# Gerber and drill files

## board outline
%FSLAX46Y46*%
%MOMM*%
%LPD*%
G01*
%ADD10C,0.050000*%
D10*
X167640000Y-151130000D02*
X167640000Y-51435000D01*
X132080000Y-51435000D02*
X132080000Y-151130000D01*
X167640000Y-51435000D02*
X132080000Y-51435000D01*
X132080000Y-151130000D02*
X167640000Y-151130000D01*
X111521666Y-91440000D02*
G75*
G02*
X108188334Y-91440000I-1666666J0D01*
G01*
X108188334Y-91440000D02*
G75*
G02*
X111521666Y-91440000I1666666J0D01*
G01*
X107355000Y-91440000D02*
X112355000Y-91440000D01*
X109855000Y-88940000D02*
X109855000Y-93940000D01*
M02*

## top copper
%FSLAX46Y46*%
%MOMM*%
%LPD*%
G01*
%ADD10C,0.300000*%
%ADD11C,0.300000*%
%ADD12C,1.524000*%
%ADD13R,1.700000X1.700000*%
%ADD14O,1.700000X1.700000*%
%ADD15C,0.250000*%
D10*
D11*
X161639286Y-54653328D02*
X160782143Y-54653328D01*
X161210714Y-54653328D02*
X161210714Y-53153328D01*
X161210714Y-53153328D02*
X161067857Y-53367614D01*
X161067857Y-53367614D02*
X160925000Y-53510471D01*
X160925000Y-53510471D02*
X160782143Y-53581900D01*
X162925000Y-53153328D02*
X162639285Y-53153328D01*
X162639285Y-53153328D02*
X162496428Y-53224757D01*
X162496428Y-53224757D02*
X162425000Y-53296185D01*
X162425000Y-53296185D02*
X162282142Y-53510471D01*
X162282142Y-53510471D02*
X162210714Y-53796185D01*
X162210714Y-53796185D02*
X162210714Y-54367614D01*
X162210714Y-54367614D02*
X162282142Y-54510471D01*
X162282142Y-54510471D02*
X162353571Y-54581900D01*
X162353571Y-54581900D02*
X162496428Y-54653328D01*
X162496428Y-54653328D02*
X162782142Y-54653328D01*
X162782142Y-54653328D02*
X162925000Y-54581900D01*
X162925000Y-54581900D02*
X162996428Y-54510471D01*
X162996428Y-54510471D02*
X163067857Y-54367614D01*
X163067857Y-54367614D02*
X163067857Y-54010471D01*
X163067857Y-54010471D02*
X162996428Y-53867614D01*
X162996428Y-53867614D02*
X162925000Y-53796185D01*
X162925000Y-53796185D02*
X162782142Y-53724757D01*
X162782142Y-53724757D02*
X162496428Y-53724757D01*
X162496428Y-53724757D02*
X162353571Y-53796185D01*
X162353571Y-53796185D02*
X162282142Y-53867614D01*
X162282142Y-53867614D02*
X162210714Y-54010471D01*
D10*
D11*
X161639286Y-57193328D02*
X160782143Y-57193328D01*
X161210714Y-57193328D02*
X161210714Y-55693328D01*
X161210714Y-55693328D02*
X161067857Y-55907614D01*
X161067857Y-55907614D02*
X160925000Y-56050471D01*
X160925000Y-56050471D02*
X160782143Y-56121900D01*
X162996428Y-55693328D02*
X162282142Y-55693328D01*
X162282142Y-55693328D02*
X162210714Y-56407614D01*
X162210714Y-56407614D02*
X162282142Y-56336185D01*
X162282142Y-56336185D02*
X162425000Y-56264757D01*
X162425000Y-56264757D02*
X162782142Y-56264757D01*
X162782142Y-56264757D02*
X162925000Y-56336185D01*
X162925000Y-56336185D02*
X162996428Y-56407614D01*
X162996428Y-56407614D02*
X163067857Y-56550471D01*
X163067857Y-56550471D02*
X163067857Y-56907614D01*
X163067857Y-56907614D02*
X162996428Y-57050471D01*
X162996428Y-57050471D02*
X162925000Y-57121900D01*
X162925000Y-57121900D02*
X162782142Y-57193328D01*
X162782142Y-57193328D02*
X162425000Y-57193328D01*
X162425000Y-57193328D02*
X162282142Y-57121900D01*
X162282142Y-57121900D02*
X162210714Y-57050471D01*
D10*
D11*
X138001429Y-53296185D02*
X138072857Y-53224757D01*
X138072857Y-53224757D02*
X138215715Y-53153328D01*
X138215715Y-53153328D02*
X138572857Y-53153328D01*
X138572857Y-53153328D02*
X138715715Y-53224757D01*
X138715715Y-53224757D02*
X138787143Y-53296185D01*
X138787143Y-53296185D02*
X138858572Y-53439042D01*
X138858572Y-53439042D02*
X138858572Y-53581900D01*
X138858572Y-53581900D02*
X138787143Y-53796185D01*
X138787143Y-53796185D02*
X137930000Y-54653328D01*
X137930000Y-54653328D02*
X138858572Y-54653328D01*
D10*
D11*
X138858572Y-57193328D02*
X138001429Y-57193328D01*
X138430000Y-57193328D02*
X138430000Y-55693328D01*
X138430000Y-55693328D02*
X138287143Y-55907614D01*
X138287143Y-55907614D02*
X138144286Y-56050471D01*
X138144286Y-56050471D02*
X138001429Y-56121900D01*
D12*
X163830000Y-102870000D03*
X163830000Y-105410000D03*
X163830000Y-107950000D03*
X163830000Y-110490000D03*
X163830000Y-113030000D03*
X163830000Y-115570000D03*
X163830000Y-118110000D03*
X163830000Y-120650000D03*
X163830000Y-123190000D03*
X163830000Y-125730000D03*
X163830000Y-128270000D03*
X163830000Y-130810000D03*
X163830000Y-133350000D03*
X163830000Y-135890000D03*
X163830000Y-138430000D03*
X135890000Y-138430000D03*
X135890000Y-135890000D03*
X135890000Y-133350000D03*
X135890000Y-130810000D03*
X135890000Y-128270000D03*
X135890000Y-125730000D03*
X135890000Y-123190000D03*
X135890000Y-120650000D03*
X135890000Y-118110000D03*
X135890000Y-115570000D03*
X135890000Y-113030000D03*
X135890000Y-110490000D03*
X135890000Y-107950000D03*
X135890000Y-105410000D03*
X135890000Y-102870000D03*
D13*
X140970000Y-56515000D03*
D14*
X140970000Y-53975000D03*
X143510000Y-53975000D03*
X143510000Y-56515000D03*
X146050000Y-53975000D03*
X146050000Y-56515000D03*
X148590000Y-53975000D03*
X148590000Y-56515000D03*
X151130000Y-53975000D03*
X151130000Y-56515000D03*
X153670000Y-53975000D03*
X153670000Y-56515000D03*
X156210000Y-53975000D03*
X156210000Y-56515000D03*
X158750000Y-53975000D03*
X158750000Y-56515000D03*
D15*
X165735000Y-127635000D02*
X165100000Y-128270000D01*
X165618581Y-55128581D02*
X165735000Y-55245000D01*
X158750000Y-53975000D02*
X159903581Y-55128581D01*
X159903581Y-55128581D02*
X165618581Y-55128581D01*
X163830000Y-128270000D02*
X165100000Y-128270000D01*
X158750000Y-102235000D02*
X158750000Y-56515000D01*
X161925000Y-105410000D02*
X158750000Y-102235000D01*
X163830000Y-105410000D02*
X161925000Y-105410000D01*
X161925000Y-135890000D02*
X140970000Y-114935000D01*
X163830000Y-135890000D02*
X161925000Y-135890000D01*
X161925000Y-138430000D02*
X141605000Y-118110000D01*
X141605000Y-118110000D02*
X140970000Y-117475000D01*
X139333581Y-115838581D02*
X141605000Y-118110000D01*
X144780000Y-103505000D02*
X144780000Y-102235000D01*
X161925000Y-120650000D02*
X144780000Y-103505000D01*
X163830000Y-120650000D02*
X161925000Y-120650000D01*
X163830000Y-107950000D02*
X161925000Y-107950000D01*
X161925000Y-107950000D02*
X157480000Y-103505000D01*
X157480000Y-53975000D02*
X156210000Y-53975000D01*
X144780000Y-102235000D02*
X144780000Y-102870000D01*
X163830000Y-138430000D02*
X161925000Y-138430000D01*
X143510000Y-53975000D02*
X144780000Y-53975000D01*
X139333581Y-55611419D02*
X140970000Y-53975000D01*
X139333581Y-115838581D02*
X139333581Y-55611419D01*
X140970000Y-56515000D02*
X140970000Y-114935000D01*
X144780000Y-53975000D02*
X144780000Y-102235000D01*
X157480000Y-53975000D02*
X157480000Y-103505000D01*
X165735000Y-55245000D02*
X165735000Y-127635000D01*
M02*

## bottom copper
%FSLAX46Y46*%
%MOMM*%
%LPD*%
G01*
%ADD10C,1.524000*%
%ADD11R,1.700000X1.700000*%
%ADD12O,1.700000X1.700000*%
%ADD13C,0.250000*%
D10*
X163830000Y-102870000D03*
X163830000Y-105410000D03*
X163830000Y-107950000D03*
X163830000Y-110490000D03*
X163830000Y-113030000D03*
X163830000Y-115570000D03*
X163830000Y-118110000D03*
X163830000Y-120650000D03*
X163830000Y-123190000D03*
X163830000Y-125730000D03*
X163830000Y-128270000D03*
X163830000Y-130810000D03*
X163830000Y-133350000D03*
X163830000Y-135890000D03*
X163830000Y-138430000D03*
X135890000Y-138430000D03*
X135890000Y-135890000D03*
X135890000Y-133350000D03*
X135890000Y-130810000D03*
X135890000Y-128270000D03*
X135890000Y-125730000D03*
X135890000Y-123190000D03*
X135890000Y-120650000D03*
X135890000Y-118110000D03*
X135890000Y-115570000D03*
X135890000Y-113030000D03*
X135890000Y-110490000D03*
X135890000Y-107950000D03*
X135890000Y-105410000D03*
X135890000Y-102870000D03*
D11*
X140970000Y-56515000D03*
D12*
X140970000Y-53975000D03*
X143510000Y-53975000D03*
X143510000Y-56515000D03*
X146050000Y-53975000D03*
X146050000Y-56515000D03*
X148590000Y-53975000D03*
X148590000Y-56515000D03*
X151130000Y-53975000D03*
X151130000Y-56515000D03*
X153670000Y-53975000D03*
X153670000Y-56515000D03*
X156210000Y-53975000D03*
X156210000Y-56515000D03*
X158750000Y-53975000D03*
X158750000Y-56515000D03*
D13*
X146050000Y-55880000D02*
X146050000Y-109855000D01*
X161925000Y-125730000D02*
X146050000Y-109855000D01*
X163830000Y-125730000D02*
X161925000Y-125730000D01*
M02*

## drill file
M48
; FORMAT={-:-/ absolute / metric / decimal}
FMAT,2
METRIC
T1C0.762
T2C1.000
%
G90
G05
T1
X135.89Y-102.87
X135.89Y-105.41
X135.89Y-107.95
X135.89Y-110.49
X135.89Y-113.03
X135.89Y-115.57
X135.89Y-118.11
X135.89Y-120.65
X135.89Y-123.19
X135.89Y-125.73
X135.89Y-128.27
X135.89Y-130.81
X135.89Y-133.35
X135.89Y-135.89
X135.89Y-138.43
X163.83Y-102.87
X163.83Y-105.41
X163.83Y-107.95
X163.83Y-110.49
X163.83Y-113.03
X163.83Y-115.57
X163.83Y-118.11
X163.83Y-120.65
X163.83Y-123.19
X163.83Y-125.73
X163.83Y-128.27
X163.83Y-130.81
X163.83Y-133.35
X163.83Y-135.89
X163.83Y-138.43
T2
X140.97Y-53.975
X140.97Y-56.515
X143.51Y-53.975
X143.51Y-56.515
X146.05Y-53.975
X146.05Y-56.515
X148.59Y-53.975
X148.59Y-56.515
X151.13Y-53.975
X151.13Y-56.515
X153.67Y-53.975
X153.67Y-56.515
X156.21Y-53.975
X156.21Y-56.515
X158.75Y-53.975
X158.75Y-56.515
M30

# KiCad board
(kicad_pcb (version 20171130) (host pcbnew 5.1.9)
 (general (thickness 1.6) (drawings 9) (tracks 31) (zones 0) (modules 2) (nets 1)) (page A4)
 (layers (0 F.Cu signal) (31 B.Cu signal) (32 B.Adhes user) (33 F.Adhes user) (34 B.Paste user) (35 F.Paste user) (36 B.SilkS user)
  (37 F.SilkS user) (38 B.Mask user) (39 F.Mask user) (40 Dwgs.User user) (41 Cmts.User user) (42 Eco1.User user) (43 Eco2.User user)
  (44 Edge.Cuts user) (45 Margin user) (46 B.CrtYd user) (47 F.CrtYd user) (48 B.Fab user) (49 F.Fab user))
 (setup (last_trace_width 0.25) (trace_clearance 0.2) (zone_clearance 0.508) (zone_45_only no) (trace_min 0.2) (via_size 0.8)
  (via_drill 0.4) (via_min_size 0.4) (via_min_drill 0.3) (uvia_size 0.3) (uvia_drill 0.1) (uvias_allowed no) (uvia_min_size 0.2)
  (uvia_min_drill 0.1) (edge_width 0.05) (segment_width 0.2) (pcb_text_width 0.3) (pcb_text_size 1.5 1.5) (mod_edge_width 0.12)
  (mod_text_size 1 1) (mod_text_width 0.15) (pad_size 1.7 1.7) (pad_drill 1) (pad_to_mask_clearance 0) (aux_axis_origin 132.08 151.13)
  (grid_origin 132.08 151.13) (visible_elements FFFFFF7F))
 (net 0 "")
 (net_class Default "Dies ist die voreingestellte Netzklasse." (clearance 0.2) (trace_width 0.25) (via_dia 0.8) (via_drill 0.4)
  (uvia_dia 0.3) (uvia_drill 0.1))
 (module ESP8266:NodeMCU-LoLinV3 (layer F.Cu) (at 149.86 123.19)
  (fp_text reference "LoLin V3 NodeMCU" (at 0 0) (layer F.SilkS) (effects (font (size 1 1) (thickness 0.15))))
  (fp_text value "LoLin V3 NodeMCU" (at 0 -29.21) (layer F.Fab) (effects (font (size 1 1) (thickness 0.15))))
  (pad 30 thru_hole circle (at 13.97 -20.32) (size 1.524 1.524) (drill 0.762) (layers *.Cu *.Mask F.SilkS))
  (pad 29 thru_hole circle (at 13.97 -17.78) (size 1.524 1.524) (drill 0.762) (layers *.Cu *.Mask F.SilkS))
  (pad 28 thru_hole circle (at 13.97 -15.24) (size 1.524 1.524) (drill 0.762) (layers *.Cu *.Mask F.SilkS))
  (pad 27 thru_hole circle (at 13.97 -12.7) (size 1.524 1.524) (drill 0.762) (layers *.Cu *.Mask F.SilkS))
  (pad 26 thru_hole circle (at 13.97 -10.16) (size 1.524 1.524) (drill 0.762) (layers *.Cu *.Mask F.SilkS))
  (pad 25 thru_hole circle (at 13.97 -7.62) (size 1.524 1.524) (drill 0.762) (layers *.Cu *.Mask F.SilkS))
  (pad 24 thru_hole circle (at 13.97 -5.08) (size 1.524 1.524) (drill 0.762) (layers *.Cu *.Mask F.SilkS))
  (pad 23 thru_hole circle (at 13.97 -2.54) (size 1.524 1.524) (drill 0.762) (layers *.Cu *.Mask F.SilkS))
  (pad 22 thru_hole circle (at 13.97 0) (size 1.524 1.524) (drill 0.762) (layers *.Cu *.Mask F.SilkS))
  (pad 21 thru_hole circle (at 13.97 2.54) (size 1.524 1.524) (drill 0.762) (layers *.Cu *.Mask F.SilkS))
  (pad 20 thru_hole circle (at 13.97 5.08) (size 1.524 1.524) (drill 0.762) (layers *.Cu *.Mask F.SilkS))
  (pad 19 thru_hole circle (at 13.97 7.62) (size 1.524 1.524) (drill 0.762) (layers *.Cu *.Mask F.SilkS))
  (pad 18 thru_hole circle (at 13.97 10.16) (size 1.524 1.524) (drill 0.762) (layers *.Cu *.Mask F.SilkS))
  (pad 17 thru_hole circle (at 13.97 12.7) (size 1.524 1.524) (drill 0.762) (layers *.Cu *.Mask F.SilkS))
  (pad 16 thru_hole circle (at 13.97 15.24) (size 1.524 1.524) (drill 0.762) (layers *.Cu *.Mask F.SilkS))
  (pad 15 thru_hole circle (at -13.97 15.24) (size 1.524 1.524) (drill 0.762) (layers *.Cu *.Mask F.SilkS))
  (pad 14 thru_hole circle (at -13.97 12.7) (size 1.524 1.524) (drill 0.762) (layers *.Cu *.Mask F.SilkS))
  (pad 13 thru_hole circle (at -13.97 10.16) (size 1.524 1.524) (drill 0.762) (layers *.Cu *.Mask F.SilkS))
  (pad 12 thru_hole circle (at -13.97 7.62) (size 1.524 1.524) (drill 0.762) (layers *.Cu *.Mask F.SilkS))
  (pad 11 thru_hole circle (at -13.97 5.08) (size 1.524 1.524) (drill 0.762) (layers *.Cu *.Mask F.SilkS))
  (pad 10 thru_hole circle (at -13.97 2.54) (size 1.524 1.524) (drill 0.762) (layers *.Cu *.Mask F.SilkS))
  (pad 9 thru_hole circle (at -13.97 0) (size 1.524 1.524) (drill 0.762) (layers *.Cu *.Mask F.SilkS))
  (pad 8 thru_hole circle (at -13.97 -2.54) (size 1.524 1.524) (drill 0.762) (layers *.Cu *.Mask F.SilkS))
  (pad 7 thru_hole circle (at -13.97 -5.08) (size 1.524 1.524) (drill 0.762) (layers *.Cu *.Mask F.SilkS))
  (pad 6 thru_hole circle (at -13.97 -7.62) (size 1.524 1.524) (drill 0.762) (layers *.Cu *.Mask F.SilkS))
  (pad 5 thru_hole circle (at -13.97 -10.16) (size 1.524 1.524) (drill 0.762) (layers *.Cu *.Mask F.SilkS))
  (pad 4 thru_hole circle (at -13.97 -12.7) (size 1.524 1.524) (drill 0.762) (layers *.Cu *.Mask F.SilkS))
  (pad 3 thru_hole circle (at -13.97 -15.24) (size 1.524 1.524) (drill 0.762) (layers *.Cu *.Mask F.SilkS))
  (pad 2 thru_hole circle (at -13.97 -17.78) (size 1.524 1.524) (drill 0.762) (layers *.Cu *.Mask F.SilkS))
  (pad 1 thru_hole circle (at -13.97 -20.32) (size 1.524 1.524) (drill 0.762) (layers *.Cu *.Mask F.SilkS)))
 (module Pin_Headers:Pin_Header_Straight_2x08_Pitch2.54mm (layer B.Cu) (at 140.97 53.975 270)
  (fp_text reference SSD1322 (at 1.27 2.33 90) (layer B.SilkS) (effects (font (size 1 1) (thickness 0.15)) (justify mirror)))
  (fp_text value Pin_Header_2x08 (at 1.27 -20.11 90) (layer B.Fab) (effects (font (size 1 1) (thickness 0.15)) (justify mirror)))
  (pad 1 thru_hole rect (at 2.54 0 270) (size 1.7 1.7) (drill 1) (layers *.Cu *.Mask))
  (pad 2 thru_hole oval (at 0 0 270) (size 1.7 1.7) (drill 1) (layers *.Cu *.Mask))
  (pad 4 thru_hole oval (at 0 -2.54 270) (size 1.7 1.7) (drill 1) (layers *.Cu *.Mask))
  (pad 3 thru_hole oval (at 2.54 -2.54 270) (size 1.7 1.7) (drill 1) (layers *.Cu *.Mask))
  (pad 6 thru_hole oval (at 0 -5.08 270) (size 1.7 1.7) (drill 1) (layers *.Cu *.Mask))
  (pad 5 thru_hole oval (at 2.54 -5.08 270) (size 1.7 1.7) (drill 1) (layers *.Cu *.Mask))
  (pad 8 thru_hole oval (at 0 -7.62 270) (size 1.7 1.7) (drill 1) (layers *.Cu *.Mask))
  (pad 7 thru_hole oval (at 2.54 -7.62 270) (size 1.7 1.7) (drill 1) (layers *.Cu *.Mask))
  (pad 10 thru_hole oval (at 0 -10.16 270) (size 1.7 1.7) (drill 1) (layers *.Cu *.Mask))
  (pad 9 thru_hole oval (at 2.54 -10.16 270) (size 1.7 1.7) (drill 1) (layers *.Cu *.Mask))
  (pad 12 thru_hole oval (at 0 -12.7 270) (size 1.7 1.7) (drill 1) (layers *.Cu *.Mask))
  (pad 11 thru_hole oval (at 2.54 -12.7 270) (size 1.7 1.7) (drill 1) (layers *.Cu *.Mask))
  (pad 14 thru_hole oval (at 0 -15.24 270) (size 1.7 1.7) (drill 1) (layers *.Cu *.Mask))
  (pad 13 thru_hole oval (at 2.54 -15.24 270) (size 1.7 1.7) (drill 1) (layers *.Cu *.Mask))
  (pad 16 thru_hole oval (at 0 -17.78 270) (size 1.7 1.7) (drill 1) (layers *.Cu *.Mask))
  (pad 15 thru_hole oval (at 2.54 -17.78 270) (size 1.7 1.7) (drill 1) (layers *.Cu *.Mask)))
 (gr_line (start 167.64 151.13) (end 167.64 51.435) (layer Edge.Cuts) (width 0.05))
 (gr_line (start 132.08 51.435) (end 132.08 151.13) (layer Edge.Cuts) (width 0.05))
 (gr_line (start 167.64 51.435) (end 132.08 51.435) (layer Edge.Cuts) (width 0.05))
 (gr_line (start 132.08 151.13) (end 167.64 151.13) (layer Edge.Cuts) (width 0.05))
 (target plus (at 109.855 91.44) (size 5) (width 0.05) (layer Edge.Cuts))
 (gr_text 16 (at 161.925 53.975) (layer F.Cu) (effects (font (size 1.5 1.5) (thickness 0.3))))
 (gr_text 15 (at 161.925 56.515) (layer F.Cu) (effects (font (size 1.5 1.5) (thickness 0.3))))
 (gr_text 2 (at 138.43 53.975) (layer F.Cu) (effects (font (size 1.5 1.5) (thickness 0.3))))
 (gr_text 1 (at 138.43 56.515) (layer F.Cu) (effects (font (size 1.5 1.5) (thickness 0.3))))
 (segment (start 165.735 127.635) (end 165.1 128.27) (width 0.25) (layer F.Cu) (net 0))
 (segment (start 165.618581 55.128581) (end 165.735 55.245) (width 0.25) (layer F.Cu) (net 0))
 (segment (start 158.75 53.975) (end 159.903581 55.128581) (width 0.25) (layer F.Cu) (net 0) (status 10))
 (segment (start 159.903581 55.128581) (end 165.618581 55.128581) (width 0.25) (layer F.Cu) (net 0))
 (segment (start 163.83 128.27) (end 165.1 128.27) (width 0.25) (layer F.Cu) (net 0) (status 10))
 (segment (start 158.75 102.235) (end 158.75 56.515) (width 0.25) (layer F.Cu) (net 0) (status 20))
 (segment (start 161.925 105.41) (end 158.75 102.235) (width 0.25) (layer F.Cu) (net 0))
 (segment (start 163.83 105.41) (end 161.925 105.41) (width 0.25) (layer F.Cu) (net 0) (status 10))
 (segment (start 161.925 135.89) (end 140.97 114.935) (width 0.25) (layer F.Cu) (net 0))
 (segment (start 163.83 135.89) (end 161.925 135.89) (width 0.25) (layer F.Cu) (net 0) (status 10))
 (segment (start 161.925 138.43) (end 141.605 118.11) (width 0.25) (layer F.Cu) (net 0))
 (segment (start 141.605 118.11) (end 140.97 117.475) (width 0.25) (layer F.Cu) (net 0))
 (segment (start 139.333581 115.838581) (end 141.605 118.11) (width 0.25) (layer F.Cu) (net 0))
 (segment (start 144.78 103.505) (end 144.78 102.235) (width 0.25) (layer F.Cu) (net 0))
 (segment (start 161.925 120.65) (end 144.78 103.505) (width 0.25) (layer F.Cu) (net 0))
 (segment (start 163.83 120.65) (end 161.925 120.65) (width 0.25) (layer F.Cu) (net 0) (status 10))
 (segment (start 146.05 55.88) (end 146.05 109.855) (width 0.25) (layer B.Cu) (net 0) (status 10))
 (segment (start 161.925 125.73) (end 146.05 109.855) (width 0.25) (layer B.Cu) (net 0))
 (segment (start 163.83 125.73) (end 161.925 125.73) (width 0.25) (layer B.Cu) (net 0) (status 10))
 (segment (start 163.83 107.95) (end 161.925 107.95) (width 0.25) (layer F.Cu) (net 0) (status 10))
 (segment (start 161.925 107.95) (end 157.48 103.505) (width 0.25) (layer F.Cu) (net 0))
 (segment (start 157.48 53.975) (end 156.21 53.975) (width 0.25) (layer F.Cu) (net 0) (status 20))
 (segment (start 144.78 102.235) (end 144.78 102.87) (width 0.25) (layer F.Cu) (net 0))
 (segment (start 163.83 138.43) (end 161.925 138.43) (width 0.25) (layer F.Cu) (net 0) (status 10))
 (segment (start 143.51 53.975) (end 144.78 53.975) (width 0.25) (layer F.Cu) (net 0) (status 10))
 (segment (start 139.333581 55.611419) (end 140.97 53.975) (width 0.25) (layer F.Cu) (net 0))
 (segment (start 139.333581 115.838581) (end 139.333581 55.611419) (width 0.25) (layer F.Cu) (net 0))
 (segment (start 140.97 56.515) (end 140.97 114.935) (width 0.25) (layer F.Cu) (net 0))
 (segment (start 144.78 53.975) (end 144.78 102.235) (width 0.25) (layer F.Cu) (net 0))
 (segment (start 157.48 53.975) (end 157.48 103.505) (width 0.25) (layer F.Cu) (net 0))
 (segment (start 165.735 55.245) (end 165.735 127.635) (width 0.25) (layer F.Cu) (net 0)))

